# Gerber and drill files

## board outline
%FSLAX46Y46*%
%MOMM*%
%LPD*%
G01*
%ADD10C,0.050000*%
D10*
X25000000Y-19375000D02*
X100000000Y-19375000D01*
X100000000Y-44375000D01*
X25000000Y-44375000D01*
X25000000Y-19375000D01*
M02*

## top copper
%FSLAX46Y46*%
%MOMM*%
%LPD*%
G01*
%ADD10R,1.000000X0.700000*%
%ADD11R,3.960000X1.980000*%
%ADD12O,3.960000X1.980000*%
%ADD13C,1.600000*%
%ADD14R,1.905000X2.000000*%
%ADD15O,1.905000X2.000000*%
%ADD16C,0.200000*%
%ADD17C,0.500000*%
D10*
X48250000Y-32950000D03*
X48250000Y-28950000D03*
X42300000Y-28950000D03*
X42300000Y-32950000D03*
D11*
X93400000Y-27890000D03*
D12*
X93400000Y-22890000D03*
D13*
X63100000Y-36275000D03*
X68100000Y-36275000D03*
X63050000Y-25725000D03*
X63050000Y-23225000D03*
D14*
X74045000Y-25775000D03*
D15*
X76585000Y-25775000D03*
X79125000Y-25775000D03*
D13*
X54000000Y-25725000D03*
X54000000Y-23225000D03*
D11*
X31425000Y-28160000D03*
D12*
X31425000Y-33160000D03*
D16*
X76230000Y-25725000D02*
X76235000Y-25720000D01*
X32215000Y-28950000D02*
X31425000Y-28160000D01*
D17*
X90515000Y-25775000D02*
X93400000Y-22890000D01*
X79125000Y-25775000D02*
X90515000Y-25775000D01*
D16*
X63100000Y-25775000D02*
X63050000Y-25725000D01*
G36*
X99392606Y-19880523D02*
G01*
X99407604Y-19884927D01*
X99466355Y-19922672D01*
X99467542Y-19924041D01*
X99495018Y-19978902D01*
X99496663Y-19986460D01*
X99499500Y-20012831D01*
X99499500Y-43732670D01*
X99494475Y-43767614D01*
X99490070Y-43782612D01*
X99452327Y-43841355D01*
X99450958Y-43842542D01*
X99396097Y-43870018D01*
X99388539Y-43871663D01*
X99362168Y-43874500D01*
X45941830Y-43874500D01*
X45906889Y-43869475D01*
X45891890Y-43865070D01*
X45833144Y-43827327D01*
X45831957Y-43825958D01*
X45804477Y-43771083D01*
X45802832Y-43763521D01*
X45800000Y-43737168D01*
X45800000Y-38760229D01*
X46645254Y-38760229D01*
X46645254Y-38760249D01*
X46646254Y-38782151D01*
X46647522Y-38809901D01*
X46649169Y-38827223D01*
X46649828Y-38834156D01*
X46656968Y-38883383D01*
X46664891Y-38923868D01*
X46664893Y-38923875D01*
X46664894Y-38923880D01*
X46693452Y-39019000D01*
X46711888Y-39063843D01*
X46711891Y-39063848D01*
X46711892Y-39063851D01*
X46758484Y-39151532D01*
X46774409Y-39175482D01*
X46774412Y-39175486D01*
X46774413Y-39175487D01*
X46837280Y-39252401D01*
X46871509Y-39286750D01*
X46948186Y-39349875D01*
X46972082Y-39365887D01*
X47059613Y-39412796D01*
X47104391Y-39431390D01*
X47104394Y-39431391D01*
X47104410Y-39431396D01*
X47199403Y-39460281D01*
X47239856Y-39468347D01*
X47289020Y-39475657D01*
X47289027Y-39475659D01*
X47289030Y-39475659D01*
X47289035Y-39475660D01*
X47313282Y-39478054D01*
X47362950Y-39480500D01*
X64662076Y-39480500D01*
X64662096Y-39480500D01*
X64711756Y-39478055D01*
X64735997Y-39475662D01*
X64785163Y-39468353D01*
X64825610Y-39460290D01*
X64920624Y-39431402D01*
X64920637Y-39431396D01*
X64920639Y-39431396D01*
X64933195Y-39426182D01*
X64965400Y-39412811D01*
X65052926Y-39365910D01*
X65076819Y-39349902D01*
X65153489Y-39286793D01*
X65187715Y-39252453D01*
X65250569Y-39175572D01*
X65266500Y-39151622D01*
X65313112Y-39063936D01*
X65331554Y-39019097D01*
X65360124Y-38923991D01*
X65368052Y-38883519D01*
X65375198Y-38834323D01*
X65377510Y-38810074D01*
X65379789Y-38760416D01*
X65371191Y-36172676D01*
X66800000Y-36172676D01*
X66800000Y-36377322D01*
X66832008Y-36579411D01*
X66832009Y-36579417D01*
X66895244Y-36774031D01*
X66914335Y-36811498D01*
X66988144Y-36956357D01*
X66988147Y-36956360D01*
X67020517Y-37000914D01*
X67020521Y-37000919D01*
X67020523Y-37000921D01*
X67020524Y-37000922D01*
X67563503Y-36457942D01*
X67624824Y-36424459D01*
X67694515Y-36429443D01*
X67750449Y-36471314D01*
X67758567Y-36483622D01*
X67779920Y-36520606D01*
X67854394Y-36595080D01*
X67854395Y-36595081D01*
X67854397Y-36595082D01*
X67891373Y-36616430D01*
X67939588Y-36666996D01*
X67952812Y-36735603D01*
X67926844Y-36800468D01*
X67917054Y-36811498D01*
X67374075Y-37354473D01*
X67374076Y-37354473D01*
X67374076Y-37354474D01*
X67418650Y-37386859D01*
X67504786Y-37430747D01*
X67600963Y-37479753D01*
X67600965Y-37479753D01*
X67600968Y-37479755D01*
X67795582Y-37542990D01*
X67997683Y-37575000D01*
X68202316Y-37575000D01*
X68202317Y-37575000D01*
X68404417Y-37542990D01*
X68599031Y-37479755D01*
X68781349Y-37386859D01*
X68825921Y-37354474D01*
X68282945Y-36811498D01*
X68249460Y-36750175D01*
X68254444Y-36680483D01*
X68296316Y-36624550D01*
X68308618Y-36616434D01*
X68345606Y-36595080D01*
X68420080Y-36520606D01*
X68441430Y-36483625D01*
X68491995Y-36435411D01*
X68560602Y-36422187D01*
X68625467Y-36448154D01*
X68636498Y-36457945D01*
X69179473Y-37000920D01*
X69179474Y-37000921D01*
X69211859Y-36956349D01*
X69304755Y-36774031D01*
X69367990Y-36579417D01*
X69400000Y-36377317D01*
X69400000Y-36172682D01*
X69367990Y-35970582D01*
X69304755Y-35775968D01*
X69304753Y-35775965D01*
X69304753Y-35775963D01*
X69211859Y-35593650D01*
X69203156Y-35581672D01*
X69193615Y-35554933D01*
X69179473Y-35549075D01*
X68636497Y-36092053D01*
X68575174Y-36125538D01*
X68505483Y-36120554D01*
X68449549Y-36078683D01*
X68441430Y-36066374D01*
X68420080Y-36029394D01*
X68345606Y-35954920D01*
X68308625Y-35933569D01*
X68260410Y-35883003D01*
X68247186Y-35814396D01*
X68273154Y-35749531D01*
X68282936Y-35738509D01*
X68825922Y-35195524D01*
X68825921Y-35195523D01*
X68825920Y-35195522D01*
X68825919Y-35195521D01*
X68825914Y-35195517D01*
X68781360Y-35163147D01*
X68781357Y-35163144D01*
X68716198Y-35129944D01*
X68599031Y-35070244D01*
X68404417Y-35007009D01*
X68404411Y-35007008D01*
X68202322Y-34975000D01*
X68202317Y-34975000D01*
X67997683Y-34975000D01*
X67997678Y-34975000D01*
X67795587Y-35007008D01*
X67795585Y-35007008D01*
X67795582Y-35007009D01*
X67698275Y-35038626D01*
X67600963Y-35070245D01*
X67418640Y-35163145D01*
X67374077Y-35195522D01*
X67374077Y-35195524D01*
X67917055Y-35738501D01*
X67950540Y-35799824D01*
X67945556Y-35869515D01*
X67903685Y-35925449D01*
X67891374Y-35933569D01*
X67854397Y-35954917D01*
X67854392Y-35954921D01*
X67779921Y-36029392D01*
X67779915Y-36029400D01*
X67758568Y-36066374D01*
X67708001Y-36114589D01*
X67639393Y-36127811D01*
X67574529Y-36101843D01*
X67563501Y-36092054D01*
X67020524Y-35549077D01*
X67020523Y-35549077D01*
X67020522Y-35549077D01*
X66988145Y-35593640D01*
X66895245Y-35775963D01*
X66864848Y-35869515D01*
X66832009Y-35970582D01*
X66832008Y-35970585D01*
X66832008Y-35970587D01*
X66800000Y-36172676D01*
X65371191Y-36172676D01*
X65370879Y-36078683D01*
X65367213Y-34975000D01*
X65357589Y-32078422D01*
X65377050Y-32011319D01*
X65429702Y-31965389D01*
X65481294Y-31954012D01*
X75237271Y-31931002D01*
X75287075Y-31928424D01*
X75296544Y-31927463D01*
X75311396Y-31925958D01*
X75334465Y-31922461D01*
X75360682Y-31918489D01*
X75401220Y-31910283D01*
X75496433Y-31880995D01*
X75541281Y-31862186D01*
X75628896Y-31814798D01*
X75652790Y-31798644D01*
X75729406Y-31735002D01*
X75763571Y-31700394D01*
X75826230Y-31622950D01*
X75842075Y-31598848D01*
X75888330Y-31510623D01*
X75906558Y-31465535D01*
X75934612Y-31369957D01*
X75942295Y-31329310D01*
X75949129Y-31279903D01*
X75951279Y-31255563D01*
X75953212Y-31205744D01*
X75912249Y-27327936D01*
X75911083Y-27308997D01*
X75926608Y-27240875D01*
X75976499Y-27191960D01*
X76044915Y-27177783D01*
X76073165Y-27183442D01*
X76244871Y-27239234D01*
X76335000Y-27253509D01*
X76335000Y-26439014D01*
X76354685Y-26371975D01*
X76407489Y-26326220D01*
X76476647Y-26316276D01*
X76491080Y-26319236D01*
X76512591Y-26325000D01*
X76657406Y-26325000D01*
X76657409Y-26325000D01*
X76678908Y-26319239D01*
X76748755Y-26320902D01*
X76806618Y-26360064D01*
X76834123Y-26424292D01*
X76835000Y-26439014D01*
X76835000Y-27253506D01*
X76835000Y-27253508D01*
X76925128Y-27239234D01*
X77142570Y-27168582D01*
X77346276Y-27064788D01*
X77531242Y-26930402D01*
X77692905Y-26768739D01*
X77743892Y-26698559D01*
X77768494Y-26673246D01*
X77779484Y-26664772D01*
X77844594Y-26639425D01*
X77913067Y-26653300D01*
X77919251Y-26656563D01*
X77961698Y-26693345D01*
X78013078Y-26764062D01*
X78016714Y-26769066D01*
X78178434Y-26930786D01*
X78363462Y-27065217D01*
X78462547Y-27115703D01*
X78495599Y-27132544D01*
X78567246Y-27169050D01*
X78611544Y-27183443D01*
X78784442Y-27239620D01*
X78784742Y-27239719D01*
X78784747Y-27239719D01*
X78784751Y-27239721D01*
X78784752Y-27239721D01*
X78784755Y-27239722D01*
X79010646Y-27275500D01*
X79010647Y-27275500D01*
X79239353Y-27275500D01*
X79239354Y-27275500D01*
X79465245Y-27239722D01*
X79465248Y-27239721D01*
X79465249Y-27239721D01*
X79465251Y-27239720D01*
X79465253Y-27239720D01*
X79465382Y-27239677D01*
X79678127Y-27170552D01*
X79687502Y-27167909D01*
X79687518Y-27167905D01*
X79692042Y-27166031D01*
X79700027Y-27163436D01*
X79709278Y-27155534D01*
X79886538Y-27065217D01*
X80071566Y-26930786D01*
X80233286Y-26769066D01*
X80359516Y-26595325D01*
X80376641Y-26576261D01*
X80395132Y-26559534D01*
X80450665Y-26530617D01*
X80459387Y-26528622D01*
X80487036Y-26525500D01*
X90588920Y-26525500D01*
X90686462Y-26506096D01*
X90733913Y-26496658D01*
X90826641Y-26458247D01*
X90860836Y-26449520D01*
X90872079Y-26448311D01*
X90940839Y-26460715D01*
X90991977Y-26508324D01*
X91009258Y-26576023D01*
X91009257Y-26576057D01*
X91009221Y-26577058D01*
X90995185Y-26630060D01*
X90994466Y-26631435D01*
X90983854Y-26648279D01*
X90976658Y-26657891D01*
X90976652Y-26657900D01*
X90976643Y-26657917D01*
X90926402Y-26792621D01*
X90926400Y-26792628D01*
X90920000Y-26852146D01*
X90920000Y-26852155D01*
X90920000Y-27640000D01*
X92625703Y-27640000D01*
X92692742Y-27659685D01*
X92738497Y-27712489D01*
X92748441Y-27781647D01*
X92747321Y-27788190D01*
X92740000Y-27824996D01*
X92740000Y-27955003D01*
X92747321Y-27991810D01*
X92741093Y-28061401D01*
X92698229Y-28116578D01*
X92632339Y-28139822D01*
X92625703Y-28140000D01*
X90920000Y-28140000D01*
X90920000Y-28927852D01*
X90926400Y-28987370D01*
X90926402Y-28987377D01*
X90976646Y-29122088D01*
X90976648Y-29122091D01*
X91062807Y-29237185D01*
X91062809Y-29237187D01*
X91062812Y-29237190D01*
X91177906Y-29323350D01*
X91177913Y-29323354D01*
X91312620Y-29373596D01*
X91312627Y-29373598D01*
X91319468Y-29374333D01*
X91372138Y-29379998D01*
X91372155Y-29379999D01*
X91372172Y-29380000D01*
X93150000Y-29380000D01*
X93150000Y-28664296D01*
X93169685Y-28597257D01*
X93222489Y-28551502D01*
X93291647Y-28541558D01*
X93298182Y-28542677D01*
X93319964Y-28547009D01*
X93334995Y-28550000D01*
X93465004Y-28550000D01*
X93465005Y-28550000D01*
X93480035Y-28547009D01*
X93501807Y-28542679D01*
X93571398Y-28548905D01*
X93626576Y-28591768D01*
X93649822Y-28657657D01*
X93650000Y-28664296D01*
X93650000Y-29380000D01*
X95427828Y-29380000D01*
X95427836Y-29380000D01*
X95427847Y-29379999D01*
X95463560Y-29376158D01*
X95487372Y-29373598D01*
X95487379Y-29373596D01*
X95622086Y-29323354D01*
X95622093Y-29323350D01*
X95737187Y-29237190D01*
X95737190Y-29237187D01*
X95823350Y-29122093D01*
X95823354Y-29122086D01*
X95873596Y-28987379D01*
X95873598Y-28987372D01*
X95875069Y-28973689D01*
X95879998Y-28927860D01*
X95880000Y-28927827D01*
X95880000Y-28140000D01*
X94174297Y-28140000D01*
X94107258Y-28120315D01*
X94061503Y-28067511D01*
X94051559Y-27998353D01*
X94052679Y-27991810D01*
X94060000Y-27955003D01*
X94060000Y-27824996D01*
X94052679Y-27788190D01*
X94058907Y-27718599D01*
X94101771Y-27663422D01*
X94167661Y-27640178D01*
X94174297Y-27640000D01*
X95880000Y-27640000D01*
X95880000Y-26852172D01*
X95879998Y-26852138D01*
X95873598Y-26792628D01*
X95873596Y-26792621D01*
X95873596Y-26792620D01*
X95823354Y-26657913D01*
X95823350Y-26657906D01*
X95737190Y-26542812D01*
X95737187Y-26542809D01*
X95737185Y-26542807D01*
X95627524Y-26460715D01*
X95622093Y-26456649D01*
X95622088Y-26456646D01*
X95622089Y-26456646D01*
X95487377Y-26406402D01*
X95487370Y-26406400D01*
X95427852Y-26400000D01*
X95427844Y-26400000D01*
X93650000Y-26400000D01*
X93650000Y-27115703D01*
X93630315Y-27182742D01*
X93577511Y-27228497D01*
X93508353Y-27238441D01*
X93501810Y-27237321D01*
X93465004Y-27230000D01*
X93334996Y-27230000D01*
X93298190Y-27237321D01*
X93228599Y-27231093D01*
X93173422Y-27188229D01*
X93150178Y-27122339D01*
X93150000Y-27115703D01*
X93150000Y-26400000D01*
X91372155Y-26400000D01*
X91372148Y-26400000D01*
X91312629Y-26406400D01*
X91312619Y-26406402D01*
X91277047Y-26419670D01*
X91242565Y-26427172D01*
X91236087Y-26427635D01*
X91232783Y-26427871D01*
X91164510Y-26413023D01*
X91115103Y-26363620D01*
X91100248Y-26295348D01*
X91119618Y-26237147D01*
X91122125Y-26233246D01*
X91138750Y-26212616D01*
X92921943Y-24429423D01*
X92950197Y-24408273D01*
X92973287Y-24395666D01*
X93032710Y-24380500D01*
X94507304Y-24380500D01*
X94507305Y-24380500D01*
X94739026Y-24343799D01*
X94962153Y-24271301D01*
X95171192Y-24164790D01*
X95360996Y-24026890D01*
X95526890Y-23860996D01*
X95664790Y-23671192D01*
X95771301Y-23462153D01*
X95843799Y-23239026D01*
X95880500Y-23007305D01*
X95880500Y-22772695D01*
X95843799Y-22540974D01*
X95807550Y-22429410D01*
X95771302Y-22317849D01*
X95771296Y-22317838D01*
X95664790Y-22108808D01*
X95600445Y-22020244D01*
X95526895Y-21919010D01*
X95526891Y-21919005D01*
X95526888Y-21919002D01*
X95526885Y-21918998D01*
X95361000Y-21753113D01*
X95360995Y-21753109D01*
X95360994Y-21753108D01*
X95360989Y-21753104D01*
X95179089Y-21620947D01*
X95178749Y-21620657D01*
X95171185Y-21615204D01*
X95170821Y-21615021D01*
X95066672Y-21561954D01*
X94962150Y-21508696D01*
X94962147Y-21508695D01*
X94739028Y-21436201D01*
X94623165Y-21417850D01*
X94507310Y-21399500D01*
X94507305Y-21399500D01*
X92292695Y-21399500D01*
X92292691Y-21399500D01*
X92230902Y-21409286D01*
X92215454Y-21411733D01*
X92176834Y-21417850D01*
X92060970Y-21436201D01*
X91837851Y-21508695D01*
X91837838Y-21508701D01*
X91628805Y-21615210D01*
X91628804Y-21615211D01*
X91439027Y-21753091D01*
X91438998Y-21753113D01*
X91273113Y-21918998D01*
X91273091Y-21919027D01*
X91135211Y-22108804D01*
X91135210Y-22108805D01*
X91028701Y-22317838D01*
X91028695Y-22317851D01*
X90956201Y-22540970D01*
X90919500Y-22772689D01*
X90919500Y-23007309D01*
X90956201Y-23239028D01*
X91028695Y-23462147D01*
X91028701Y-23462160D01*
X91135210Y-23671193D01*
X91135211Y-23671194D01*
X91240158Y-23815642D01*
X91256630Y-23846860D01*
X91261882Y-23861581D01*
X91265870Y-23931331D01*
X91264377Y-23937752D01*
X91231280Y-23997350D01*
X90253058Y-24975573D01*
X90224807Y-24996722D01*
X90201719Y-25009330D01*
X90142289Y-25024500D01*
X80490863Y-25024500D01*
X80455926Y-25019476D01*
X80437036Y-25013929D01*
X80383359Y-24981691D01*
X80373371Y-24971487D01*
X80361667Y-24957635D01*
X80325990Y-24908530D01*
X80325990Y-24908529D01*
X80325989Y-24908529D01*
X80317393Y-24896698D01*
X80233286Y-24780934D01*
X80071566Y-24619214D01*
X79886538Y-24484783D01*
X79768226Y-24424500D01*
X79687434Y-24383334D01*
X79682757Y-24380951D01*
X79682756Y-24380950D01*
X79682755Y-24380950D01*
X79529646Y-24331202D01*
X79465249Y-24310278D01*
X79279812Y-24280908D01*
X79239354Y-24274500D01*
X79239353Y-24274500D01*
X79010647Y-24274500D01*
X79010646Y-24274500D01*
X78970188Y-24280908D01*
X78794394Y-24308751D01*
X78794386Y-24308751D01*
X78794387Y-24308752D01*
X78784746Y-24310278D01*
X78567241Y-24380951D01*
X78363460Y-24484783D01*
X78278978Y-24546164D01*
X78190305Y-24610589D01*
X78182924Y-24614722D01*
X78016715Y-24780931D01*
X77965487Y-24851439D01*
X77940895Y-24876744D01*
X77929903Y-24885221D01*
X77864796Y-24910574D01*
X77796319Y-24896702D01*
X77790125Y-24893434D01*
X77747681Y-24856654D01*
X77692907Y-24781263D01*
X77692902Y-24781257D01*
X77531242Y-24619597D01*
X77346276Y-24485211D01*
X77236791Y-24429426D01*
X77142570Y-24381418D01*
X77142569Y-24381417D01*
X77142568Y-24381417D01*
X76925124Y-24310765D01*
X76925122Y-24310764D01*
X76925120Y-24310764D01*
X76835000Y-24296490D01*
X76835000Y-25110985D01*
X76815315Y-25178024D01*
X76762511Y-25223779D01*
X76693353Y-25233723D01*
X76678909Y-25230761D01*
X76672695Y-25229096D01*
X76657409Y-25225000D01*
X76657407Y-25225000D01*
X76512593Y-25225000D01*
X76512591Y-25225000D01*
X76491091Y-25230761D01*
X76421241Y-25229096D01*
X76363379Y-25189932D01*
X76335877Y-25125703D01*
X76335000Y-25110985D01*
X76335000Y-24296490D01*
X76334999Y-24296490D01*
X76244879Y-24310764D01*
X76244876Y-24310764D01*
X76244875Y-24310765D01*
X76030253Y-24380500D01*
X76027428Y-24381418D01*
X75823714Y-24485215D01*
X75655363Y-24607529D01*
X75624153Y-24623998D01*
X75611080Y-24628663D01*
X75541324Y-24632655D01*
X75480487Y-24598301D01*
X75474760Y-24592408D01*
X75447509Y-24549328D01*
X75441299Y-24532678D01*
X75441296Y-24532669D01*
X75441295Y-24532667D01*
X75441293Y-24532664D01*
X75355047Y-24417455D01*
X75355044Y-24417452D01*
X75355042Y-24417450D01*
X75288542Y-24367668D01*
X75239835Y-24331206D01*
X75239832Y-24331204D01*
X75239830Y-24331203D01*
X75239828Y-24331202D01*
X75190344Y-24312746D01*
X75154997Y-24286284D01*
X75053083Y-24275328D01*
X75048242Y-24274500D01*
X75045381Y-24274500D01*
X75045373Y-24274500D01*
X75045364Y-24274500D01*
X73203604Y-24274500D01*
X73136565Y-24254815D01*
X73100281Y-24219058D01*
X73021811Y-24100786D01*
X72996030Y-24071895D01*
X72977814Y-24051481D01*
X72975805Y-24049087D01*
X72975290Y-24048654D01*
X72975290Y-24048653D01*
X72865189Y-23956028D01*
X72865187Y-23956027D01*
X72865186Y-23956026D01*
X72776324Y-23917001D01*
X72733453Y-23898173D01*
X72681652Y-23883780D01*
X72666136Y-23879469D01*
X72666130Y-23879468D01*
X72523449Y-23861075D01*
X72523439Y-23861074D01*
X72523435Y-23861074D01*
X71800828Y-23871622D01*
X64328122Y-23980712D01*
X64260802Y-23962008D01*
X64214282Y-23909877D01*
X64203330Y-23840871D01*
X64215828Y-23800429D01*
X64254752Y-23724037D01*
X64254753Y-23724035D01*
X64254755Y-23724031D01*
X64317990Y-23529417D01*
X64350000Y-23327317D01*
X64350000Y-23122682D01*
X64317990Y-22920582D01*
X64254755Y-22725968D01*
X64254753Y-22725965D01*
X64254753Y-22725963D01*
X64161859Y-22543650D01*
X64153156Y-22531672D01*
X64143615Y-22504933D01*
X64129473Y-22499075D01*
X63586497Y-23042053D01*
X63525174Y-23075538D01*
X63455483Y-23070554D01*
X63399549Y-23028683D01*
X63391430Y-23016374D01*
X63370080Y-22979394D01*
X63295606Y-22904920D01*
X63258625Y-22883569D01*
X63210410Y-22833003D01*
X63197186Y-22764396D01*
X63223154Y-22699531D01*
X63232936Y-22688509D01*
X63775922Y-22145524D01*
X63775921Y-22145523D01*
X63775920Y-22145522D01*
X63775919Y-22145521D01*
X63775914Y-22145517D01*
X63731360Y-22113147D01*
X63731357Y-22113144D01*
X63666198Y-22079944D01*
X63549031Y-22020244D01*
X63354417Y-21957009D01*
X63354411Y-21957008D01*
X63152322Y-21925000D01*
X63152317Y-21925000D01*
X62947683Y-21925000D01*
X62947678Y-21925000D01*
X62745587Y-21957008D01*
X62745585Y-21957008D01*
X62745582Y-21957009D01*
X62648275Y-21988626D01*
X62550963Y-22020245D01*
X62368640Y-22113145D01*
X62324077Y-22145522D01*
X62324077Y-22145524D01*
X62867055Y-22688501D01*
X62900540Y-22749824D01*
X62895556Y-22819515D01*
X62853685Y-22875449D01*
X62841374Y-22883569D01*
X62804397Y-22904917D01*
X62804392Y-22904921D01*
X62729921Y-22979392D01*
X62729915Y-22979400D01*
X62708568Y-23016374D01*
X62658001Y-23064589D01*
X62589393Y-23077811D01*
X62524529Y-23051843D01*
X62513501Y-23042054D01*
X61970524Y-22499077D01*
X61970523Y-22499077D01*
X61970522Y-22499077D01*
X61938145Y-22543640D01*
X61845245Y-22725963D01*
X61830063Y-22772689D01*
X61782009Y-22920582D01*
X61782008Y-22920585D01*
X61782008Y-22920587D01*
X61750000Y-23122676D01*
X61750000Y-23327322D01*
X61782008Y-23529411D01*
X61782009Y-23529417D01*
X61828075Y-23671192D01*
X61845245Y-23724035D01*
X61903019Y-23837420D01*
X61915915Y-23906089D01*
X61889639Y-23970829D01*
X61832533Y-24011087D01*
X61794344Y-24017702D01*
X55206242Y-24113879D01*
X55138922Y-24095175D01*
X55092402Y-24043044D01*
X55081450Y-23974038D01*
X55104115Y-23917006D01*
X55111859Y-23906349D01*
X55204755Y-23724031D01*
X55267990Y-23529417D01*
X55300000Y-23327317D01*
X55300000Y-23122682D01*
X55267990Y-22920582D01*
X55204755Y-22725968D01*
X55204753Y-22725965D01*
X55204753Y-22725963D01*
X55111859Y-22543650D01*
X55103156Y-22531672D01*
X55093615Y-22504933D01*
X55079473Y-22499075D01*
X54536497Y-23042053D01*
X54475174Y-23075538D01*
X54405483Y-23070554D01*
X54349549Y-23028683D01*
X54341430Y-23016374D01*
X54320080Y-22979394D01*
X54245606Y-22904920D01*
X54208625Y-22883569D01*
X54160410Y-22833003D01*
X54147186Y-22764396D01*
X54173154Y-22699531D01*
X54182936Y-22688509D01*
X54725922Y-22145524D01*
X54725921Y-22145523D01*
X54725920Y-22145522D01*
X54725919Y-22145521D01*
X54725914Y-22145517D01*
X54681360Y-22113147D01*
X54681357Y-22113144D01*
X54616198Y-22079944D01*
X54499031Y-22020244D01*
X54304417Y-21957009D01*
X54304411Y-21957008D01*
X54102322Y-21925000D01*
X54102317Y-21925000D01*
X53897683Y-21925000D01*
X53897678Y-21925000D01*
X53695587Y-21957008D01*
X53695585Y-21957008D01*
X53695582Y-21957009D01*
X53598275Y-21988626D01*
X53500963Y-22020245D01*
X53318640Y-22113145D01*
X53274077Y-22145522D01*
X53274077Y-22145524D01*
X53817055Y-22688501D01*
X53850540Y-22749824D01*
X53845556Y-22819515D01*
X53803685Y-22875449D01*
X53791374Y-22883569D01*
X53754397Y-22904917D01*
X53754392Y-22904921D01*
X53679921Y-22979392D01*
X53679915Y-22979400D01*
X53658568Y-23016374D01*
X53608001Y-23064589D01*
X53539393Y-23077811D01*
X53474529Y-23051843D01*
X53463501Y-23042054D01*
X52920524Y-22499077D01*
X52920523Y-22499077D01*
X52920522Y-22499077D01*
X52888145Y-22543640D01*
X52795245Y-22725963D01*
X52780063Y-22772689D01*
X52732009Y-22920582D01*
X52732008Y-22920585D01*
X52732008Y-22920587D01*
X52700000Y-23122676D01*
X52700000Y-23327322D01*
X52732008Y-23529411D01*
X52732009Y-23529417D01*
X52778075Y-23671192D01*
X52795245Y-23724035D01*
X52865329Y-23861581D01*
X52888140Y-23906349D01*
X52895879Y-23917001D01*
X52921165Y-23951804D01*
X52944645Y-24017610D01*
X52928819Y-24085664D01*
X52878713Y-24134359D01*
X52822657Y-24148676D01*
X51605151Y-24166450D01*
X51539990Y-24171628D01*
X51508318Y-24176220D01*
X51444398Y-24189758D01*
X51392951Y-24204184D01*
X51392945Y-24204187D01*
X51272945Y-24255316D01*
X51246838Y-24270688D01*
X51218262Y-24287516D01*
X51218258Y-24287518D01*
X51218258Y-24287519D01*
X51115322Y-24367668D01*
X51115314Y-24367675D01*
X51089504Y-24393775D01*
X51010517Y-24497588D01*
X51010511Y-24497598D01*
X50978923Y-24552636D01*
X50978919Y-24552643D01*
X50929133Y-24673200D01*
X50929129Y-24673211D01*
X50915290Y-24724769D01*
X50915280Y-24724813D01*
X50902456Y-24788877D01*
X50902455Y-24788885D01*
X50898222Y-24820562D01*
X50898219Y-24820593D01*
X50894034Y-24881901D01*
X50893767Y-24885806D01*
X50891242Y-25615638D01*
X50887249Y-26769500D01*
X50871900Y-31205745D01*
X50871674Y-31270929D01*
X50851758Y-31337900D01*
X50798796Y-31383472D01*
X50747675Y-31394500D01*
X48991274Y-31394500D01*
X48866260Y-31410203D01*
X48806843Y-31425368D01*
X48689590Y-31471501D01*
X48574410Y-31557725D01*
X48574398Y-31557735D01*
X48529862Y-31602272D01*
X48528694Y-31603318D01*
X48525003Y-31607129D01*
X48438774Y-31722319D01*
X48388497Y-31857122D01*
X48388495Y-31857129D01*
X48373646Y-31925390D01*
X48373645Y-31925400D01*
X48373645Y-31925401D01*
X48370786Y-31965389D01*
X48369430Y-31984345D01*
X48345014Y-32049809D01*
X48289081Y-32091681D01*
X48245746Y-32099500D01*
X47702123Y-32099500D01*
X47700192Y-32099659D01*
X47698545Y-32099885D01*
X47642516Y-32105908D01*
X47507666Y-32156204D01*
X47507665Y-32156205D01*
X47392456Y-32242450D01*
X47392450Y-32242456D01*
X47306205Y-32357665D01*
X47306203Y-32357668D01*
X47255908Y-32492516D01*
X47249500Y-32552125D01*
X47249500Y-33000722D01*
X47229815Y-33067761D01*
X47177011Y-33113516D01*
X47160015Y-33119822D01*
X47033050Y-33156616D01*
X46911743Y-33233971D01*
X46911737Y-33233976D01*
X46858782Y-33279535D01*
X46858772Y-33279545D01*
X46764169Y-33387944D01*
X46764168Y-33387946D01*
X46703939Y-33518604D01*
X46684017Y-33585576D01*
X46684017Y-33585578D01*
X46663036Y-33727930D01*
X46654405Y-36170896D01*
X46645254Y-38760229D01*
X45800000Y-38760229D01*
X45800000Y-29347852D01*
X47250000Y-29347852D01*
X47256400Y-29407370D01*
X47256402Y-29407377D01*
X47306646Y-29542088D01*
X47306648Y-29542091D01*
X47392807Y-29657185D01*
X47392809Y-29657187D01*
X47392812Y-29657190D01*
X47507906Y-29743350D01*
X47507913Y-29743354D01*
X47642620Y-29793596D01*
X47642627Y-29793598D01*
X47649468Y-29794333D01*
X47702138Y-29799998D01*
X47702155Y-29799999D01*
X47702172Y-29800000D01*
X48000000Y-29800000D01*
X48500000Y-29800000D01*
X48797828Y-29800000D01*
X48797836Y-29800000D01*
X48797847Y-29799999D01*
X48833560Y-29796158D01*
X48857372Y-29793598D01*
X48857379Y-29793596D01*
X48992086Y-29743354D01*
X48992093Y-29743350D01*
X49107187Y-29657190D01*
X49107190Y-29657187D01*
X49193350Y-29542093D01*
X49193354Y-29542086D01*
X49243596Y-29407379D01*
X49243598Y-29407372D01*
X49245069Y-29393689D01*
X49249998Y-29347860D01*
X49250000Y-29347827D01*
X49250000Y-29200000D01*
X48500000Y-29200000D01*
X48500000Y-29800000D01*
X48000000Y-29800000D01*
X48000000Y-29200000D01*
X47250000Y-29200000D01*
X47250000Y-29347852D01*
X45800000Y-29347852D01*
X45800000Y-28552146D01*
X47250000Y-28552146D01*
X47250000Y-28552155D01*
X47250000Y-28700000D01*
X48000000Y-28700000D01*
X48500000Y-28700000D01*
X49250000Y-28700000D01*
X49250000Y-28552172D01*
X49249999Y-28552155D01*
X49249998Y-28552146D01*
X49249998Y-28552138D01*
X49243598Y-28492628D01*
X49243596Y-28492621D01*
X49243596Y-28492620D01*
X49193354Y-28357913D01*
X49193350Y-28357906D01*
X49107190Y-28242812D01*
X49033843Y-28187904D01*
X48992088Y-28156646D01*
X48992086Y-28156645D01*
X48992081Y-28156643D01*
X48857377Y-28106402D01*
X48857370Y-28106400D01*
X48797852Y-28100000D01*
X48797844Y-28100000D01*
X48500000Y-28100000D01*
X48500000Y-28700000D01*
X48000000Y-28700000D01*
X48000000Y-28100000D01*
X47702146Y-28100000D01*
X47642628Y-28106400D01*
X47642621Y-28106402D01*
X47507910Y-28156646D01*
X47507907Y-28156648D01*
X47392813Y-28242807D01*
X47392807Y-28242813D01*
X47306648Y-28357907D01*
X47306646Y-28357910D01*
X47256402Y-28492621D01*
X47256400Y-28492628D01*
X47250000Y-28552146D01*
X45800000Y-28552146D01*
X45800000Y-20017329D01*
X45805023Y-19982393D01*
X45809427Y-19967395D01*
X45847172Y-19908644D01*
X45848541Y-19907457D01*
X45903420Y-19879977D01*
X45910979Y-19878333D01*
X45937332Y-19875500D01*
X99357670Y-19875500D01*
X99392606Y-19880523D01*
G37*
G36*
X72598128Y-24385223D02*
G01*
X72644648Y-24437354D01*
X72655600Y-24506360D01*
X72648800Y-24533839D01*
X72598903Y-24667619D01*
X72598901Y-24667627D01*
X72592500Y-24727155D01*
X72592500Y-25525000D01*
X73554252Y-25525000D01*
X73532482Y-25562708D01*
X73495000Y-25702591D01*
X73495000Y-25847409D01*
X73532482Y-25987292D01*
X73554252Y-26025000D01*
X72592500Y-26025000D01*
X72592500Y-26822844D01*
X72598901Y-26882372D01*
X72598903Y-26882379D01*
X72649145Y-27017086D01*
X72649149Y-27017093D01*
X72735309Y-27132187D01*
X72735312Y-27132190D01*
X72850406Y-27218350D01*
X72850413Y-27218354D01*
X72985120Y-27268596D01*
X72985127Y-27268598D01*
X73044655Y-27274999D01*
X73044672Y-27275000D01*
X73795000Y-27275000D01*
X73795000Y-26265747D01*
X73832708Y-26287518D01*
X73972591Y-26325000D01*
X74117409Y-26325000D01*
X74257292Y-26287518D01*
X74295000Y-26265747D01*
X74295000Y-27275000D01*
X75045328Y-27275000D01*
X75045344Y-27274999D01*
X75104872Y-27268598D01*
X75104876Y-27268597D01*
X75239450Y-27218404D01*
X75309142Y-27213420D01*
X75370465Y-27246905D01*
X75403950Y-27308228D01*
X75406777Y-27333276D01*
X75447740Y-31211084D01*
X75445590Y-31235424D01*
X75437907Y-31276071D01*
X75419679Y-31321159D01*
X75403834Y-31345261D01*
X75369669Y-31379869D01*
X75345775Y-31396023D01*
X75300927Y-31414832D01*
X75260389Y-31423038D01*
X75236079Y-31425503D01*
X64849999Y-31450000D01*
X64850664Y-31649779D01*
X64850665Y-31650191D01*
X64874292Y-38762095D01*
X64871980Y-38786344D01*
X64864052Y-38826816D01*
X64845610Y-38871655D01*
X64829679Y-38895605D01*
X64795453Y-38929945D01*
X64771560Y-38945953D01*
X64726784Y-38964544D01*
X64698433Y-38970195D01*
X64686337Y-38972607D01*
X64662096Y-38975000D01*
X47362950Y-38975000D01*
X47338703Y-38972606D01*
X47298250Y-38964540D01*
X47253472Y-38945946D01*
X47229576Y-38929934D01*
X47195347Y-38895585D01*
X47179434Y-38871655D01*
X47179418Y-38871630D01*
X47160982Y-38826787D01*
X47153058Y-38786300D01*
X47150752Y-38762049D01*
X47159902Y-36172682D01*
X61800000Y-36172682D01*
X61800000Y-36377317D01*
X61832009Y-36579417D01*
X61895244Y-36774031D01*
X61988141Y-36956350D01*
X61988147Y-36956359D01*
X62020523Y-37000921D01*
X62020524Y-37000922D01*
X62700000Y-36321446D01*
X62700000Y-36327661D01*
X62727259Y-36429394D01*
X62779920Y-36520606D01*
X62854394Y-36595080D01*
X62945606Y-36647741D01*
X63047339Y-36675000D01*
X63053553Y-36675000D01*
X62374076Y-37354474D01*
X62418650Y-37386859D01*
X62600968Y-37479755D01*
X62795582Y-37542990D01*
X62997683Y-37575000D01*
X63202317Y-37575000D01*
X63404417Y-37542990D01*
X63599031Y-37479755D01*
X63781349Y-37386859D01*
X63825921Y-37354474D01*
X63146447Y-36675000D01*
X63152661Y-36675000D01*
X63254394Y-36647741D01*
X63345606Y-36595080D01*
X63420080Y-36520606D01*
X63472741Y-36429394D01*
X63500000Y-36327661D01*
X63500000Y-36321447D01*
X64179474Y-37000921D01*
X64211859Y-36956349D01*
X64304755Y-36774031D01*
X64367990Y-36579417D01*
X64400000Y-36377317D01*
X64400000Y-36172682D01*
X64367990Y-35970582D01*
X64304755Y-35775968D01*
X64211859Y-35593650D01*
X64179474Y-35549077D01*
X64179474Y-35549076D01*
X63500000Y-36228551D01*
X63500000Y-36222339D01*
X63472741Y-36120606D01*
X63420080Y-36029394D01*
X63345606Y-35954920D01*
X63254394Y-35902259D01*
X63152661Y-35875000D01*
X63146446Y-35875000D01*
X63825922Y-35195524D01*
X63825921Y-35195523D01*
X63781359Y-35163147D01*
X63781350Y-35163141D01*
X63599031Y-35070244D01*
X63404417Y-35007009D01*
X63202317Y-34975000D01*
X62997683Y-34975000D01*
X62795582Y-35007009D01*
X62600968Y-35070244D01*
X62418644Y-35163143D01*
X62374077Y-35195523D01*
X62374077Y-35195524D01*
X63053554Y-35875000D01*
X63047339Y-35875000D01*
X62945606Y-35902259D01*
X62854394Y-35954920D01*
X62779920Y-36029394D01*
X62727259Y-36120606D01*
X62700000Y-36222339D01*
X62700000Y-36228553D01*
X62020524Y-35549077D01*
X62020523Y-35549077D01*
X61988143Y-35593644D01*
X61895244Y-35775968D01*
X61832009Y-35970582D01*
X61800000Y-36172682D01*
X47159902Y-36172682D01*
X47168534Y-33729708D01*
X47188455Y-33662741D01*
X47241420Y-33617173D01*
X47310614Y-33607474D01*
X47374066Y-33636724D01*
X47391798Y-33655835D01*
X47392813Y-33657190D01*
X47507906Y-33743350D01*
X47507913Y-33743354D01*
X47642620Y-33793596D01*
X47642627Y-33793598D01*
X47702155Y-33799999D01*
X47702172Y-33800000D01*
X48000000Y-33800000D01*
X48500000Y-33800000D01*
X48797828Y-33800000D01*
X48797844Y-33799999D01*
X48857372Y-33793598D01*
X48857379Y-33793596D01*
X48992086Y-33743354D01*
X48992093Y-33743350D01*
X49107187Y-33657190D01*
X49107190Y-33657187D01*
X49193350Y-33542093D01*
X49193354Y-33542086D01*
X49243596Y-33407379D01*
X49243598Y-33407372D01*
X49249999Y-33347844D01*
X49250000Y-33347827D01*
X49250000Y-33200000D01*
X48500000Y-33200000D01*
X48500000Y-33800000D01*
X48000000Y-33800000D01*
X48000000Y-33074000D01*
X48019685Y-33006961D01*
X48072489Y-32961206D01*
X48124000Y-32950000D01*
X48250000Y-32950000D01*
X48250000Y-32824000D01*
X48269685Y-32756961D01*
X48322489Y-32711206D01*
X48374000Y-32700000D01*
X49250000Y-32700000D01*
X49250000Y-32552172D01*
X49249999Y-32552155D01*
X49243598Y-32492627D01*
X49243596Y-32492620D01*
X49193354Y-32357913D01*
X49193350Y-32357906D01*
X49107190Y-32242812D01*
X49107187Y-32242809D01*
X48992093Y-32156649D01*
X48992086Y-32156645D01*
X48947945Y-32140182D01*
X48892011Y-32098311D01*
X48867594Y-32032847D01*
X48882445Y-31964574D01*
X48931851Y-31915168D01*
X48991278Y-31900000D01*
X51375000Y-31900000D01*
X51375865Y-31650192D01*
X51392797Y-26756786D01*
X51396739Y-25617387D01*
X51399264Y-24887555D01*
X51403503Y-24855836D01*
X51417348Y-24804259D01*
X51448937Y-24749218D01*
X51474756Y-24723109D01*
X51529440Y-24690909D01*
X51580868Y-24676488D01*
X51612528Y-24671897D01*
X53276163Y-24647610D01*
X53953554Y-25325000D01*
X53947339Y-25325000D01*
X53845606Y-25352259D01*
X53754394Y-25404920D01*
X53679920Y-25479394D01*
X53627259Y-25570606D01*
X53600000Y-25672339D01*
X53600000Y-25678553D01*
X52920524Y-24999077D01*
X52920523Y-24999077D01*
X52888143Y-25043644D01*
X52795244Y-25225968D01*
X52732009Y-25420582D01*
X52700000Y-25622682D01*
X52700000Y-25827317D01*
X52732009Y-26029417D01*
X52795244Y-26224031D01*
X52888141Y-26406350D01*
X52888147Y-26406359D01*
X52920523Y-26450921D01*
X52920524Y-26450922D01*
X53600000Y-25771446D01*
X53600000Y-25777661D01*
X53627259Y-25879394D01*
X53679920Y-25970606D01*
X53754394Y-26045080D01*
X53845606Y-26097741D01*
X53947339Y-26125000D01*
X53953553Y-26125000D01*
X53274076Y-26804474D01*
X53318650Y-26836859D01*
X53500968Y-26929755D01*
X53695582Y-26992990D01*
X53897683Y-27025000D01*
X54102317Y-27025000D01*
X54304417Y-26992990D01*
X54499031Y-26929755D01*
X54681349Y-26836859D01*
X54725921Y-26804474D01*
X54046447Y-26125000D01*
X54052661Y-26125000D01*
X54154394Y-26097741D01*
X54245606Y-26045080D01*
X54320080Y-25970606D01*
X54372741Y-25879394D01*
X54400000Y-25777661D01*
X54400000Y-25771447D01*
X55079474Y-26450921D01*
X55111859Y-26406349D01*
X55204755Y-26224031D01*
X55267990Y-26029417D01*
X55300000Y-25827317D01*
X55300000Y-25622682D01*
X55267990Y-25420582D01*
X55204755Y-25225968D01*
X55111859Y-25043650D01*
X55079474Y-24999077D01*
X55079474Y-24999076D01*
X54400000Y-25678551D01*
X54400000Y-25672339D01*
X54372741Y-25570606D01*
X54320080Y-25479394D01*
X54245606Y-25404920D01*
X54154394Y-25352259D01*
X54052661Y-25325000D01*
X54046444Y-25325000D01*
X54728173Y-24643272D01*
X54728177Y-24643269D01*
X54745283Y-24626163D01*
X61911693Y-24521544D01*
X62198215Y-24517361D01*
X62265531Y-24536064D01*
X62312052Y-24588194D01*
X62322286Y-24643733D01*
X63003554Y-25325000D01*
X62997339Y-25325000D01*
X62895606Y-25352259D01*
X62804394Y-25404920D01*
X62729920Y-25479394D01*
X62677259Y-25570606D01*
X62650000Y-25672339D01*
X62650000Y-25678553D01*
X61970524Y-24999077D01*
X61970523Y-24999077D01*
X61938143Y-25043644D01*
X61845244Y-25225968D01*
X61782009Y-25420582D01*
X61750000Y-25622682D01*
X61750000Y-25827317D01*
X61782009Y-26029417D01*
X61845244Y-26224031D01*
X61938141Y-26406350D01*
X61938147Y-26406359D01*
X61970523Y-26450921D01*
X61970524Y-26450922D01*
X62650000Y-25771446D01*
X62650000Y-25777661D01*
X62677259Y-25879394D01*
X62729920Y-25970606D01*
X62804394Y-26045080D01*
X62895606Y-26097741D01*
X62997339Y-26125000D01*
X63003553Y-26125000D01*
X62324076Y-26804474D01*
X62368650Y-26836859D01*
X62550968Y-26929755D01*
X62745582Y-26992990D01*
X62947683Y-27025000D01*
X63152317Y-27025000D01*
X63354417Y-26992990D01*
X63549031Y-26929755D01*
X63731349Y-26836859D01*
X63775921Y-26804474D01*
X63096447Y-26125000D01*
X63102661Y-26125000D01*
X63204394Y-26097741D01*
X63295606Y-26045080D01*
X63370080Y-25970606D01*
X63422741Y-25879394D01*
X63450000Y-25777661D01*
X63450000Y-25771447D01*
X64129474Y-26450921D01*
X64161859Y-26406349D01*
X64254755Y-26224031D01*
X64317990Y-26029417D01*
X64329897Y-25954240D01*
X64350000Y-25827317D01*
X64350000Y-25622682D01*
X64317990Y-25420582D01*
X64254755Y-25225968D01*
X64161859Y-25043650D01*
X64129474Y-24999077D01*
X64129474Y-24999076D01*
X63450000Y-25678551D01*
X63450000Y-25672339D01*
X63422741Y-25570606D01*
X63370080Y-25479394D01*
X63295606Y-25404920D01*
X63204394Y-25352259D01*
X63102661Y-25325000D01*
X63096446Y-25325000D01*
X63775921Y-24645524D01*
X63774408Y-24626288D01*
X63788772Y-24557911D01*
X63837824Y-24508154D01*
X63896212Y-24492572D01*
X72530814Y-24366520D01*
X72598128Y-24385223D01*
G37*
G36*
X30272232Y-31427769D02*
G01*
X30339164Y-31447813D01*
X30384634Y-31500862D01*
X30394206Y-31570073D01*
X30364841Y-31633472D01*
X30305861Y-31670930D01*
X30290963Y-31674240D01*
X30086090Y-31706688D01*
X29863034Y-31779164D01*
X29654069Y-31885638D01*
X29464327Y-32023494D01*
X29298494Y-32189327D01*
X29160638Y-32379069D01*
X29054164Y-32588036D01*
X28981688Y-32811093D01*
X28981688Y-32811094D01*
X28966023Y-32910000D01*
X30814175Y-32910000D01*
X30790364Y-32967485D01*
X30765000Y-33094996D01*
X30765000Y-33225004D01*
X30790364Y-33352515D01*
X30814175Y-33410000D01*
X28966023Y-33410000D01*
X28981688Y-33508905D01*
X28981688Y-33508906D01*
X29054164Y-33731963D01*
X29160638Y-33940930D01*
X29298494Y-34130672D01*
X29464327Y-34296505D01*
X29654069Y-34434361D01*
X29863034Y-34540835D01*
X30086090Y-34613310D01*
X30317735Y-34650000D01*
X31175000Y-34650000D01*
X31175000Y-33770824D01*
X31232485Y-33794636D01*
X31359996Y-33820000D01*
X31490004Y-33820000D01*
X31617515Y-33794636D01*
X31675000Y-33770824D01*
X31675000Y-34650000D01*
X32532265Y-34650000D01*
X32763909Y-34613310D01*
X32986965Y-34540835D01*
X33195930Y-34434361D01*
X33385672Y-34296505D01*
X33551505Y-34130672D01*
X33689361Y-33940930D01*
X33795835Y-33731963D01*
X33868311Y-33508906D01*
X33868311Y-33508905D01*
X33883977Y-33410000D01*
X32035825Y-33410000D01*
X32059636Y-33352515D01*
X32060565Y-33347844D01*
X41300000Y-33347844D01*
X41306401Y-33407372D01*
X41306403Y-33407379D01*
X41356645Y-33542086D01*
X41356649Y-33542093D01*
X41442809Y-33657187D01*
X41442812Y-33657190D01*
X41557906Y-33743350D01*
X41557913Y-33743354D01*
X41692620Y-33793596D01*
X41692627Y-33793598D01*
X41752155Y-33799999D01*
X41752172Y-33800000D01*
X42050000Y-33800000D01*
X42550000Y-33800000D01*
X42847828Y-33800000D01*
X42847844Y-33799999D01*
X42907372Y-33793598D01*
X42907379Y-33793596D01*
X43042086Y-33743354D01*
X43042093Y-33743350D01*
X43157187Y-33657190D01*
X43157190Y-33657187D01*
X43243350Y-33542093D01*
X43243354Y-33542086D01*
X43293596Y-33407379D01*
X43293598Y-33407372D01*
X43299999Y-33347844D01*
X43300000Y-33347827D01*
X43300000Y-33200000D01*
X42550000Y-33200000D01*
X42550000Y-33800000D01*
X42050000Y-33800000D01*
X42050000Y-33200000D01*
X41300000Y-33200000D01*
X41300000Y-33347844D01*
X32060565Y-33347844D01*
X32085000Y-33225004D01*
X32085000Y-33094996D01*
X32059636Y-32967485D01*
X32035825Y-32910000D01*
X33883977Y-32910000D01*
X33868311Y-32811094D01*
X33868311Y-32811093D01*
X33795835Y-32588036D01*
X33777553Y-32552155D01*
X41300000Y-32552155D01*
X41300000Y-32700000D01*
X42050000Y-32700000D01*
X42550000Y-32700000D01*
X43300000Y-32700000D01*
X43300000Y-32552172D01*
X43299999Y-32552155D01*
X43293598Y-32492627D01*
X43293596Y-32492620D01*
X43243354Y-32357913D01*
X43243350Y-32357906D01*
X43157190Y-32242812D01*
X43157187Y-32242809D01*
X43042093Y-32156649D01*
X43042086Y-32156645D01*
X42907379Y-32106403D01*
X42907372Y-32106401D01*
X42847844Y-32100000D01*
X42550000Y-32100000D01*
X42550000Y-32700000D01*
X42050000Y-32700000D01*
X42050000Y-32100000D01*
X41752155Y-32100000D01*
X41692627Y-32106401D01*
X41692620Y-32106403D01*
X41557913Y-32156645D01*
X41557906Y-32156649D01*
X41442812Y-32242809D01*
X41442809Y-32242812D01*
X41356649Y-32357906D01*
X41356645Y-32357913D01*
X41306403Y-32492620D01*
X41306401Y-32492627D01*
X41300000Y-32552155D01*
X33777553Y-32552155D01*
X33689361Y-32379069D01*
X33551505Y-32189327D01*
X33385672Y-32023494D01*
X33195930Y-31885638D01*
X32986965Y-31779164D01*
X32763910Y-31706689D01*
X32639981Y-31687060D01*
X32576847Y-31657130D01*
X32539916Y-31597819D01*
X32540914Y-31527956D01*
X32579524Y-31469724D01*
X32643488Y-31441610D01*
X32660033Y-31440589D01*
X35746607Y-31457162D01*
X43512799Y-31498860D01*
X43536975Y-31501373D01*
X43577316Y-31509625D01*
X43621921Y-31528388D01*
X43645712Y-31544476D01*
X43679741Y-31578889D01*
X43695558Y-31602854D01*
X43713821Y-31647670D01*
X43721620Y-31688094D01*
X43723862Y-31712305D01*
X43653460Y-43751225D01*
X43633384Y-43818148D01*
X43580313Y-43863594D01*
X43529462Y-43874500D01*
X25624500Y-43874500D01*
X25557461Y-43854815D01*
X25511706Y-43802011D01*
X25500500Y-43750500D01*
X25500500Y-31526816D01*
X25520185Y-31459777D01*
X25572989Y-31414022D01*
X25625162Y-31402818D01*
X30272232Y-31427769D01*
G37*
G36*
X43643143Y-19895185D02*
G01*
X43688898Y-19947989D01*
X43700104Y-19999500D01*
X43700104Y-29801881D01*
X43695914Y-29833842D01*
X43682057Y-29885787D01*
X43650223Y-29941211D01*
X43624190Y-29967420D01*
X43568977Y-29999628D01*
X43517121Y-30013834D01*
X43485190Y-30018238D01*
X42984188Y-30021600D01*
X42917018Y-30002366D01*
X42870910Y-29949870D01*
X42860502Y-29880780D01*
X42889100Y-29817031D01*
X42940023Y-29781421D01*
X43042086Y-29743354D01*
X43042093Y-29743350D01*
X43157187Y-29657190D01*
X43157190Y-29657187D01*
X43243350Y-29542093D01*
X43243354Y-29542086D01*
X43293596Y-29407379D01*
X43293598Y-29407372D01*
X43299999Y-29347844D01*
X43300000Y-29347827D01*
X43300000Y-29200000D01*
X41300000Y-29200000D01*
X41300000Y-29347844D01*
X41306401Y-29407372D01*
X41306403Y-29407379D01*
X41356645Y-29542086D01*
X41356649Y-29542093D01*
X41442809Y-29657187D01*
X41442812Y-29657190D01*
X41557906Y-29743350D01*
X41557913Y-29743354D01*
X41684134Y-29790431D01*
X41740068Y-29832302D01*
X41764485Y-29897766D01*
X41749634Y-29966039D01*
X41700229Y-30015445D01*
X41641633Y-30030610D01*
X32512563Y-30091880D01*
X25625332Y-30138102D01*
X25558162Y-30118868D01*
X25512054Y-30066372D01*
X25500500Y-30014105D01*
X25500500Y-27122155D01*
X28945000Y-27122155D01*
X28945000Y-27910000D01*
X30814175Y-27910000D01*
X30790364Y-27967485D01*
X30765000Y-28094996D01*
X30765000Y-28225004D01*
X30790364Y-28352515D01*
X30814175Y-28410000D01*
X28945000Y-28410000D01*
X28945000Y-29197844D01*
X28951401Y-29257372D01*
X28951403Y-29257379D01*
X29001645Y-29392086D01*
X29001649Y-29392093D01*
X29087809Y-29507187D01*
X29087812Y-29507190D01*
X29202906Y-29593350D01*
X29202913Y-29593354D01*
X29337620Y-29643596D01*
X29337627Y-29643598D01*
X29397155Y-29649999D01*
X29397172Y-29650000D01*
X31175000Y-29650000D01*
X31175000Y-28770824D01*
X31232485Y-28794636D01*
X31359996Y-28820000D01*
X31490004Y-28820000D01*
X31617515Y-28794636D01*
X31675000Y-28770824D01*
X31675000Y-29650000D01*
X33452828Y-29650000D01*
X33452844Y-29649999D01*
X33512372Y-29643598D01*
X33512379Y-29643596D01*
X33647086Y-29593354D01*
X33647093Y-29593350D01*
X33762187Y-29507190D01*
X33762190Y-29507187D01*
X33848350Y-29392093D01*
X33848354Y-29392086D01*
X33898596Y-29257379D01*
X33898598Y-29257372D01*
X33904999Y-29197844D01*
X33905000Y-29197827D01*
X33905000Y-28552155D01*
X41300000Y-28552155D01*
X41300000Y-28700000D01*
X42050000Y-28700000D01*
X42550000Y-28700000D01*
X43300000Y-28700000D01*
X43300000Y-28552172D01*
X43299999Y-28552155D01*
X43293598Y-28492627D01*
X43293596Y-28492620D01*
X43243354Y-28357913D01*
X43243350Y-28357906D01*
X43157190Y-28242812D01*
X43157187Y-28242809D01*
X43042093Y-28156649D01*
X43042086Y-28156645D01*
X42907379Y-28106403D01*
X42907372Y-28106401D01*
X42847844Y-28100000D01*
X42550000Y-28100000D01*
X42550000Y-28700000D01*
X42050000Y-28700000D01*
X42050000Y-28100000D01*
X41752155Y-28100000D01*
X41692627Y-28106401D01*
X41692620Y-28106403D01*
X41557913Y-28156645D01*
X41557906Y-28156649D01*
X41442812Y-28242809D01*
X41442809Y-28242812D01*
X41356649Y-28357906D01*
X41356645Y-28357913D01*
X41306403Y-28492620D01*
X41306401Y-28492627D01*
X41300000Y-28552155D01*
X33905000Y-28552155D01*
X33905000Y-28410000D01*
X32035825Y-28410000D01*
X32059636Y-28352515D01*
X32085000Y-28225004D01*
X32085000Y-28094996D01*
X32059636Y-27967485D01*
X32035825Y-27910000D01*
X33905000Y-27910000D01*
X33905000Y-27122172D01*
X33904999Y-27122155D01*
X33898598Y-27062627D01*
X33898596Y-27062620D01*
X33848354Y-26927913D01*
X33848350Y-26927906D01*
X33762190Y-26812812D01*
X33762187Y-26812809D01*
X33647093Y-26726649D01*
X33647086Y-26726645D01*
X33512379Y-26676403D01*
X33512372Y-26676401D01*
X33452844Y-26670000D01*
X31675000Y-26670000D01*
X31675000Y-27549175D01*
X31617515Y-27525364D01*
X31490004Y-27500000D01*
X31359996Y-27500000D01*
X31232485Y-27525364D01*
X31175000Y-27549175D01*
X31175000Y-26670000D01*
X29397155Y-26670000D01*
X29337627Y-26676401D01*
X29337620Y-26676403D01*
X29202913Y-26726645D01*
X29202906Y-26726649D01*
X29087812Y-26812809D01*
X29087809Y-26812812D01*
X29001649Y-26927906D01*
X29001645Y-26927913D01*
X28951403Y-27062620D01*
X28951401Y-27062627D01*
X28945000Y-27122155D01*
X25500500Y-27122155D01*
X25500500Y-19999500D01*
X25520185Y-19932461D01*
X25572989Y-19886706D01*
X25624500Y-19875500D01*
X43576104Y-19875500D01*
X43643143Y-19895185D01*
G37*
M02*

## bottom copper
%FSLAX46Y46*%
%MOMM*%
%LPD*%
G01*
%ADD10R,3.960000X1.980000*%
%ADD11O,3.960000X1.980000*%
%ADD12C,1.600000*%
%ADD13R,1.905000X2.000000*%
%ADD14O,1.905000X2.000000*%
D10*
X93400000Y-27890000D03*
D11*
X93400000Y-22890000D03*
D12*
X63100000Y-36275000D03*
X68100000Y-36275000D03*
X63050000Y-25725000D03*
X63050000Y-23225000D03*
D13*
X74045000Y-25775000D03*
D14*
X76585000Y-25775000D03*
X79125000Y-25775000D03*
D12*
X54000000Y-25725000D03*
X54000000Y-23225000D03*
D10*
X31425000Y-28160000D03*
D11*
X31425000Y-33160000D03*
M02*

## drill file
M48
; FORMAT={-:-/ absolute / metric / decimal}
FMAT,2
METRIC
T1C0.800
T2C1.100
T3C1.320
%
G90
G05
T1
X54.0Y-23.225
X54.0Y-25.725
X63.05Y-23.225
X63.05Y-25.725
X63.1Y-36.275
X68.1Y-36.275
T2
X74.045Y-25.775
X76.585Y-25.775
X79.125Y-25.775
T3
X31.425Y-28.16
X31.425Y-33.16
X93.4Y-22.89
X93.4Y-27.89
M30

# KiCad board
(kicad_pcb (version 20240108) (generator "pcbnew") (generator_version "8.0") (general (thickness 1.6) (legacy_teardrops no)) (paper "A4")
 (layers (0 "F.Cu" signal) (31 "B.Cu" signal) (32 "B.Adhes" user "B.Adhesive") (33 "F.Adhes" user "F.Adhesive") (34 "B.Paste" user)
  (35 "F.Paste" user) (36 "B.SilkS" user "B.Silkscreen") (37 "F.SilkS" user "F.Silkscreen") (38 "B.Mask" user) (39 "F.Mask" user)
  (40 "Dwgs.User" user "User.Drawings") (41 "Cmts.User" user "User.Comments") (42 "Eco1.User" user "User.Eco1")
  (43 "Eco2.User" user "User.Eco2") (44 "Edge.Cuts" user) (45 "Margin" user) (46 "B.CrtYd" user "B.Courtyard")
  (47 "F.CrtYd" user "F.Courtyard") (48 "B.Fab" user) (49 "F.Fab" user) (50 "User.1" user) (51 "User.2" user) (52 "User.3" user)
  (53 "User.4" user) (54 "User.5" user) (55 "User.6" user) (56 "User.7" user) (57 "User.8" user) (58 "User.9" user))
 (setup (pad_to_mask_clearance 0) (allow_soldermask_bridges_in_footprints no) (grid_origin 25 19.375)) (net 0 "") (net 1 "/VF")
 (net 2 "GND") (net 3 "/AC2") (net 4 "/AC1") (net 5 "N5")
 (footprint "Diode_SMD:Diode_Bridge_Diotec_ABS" (layer "F.Cu") (at 45.275 30.95 180)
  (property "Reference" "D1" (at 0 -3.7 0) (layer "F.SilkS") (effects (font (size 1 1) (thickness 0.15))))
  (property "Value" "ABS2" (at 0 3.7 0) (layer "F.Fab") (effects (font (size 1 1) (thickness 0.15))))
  (pad "1" smd rect (at -2.975 -2 180) (size 1 0.7) (layers "F.Cu" "F.Paste" "F.Mask") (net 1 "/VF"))
  (pad "2" smd rect (at -2.975 2 180) (size 1 0.7) (layers "F.Cu" "F.Paste" "F.Mask") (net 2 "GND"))
  (pad "3" smd rect (at 2.975 2 180) (size 1 0.7) (layers "F.Cu" "F.Paste" "F.Mask") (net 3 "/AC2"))
  (pad "4" smd rect (at 2.975 -2 180) (size 1 0.7) (layers "F.Cu" "F.Paste" "F.Mask") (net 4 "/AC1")))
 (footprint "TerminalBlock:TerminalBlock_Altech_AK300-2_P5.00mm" (layer "F.Cu") (at 93.4 27.89 90)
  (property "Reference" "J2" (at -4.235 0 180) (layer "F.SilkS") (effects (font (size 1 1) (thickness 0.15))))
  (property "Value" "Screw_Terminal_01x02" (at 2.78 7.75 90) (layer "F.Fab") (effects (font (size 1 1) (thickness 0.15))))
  (pad "1" thru_hole rect (at 0 0 90) (size 1.98 3.96) (drill 1.32) (layers "*.Cu" "*.Mask") (remove_unused_layers no) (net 2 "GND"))
  (pad "2" thru_hole oval (at 5 0 90) (size 1.98 3.96) (drill 1.32) (layers "*.Cu" "*.Mask") (remove_unused_layers no) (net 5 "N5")))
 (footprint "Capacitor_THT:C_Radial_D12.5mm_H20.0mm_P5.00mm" (layer "F.Cu") (at 63.1 36.275)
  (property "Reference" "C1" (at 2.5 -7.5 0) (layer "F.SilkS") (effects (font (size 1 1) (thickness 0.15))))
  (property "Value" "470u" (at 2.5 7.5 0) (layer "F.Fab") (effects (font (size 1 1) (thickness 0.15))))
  (pad "1" thru_hole circle (at 0 0) (size 1.6 1.6) (drill 0.8) (layers "*.Cu" "*.Mask") (remove_unused_layers no) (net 1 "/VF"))
  (pad "2" thru_hole circle (at 5 0) (size 1.6 1.6) (drill 0.8) (layers "*.Cu" "*.Mask") (remove_unused_layers no) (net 2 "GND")))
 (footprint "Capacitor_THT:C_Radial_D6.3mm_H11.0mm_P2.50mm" (layer "F.Cu") (at 63.05 25.725 90)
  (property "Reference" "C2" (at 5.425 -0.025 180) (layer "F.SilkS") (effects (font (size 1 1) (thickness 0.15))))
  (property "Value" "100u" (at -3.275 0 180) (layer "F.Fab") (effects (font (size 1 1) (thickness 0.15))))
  (pad "1" thru_hole circle (at 0 0 90) (size 1.6 1.6) (drill 0.8) (layers "*.Cu" "*.Mask") (remove_unused_layers no) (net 1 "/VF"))
  (pad "2" thru_hole circle (at 2.5 0 90) (size 1.6 1.6) (drill 0.8) (layers "*.Cu" "*.Mask") (remove_unused_layers no) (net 2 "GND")))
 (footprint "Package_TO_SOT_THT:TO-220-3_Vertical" (layer "F.Cu") (at 74.045 25.775)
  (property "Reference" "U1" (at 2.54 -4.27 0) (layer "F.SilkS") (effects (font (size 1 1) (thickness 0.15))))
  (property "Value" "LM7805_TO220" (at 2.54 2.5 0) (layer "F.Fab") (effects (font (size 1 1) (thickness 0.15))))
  (pad "1" thru_hole rect (at 0 0) (size 1.905 2) (drill 1.1) (layers "*.Cu" "*.Mask") (remove_unused_layers no) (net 1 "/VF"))
  (pad "2" thru_hole oval (at 2.54 0) (size 1.905 2) (drill 1.1) (layers "*.Cu" "*.Mask") (remove_unused_layers no) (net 2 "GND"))
  (pad "3" thru_hole oval (at 5.08 0) (size 1.905 2) (drill 1.1) (layers "*.Cu" "*.Mask") (remove_unused_layers no) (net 5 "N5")))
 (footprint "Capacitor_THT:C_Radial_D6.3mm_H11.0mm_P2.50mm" (layer "F.Cu") (at 54 25.725 90)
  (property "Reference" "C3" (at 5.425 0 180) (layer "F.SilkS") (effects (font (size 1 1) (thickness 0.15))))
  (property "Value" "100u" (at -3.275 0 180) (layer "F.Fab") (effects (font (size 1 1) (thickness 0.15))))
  (pad "1" thru_hole circle (at 0 0 90) (size 1.6 1.6) (drill 0.8) (layers "*.Cu" "*.Mask") (remove_unused_layers no) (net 1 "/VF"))
  (pad "2" thru_hole circle (at 2.5 0 90) (size 1.6 1.6) (drill 0.8) (layers "*.Cu" "*.Mask") (remove_unused_layers no) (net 2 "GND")))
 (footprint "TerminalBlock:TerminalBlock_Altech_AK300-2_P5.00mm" (layer "F.Cu") (at 31.425 28.16 -90)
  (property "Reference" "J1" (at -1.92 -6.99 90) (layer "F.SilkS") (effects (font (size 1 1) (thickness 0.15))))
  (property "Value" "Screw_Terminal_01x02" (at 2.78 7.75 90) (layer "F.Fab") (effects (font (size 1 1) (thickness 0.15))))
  (pad "1" thru_hole rect (at 0 0 270) (size 1.98 3.96) (drill 1.32) (layers "*.Cu" "*.Mask") (remove_unused_layers no) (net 3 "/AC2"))
  (pad "2" thru_hole oval (at 5 0 270) (size 1.98 3.96) (drill 1.32) (layers "*.Cu" "*.Mask") (remove_unused_layers no) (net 4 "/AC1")))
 (gr_rect (start 25 19.375) (end 100 44.375) (stroke (width 0.05) (type default)) (fill none) (layer "Edge.Cuts"))
 (segment (start 76.23 25.725) (end 76.235 25.72) (width 0.2) (layer "F.Cu") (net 2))
 (segment (start 32.215 28.95) (end 31.425 28.16) (width 0.2) (layer "F.Cu") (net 3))
 (segment (start 90.515 25.775) (end 93.4 22.89) (width 0.5) (layer "F.Cu") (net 5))
 (segment (start 79.125 25.775) (end 90.515 25.775) (width 0.5) (layer "F.Cu") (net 5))
 (segment (start 63.1 25.775) (end 63.05 25.725) (width 0.2) (layer "F.Cu") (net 1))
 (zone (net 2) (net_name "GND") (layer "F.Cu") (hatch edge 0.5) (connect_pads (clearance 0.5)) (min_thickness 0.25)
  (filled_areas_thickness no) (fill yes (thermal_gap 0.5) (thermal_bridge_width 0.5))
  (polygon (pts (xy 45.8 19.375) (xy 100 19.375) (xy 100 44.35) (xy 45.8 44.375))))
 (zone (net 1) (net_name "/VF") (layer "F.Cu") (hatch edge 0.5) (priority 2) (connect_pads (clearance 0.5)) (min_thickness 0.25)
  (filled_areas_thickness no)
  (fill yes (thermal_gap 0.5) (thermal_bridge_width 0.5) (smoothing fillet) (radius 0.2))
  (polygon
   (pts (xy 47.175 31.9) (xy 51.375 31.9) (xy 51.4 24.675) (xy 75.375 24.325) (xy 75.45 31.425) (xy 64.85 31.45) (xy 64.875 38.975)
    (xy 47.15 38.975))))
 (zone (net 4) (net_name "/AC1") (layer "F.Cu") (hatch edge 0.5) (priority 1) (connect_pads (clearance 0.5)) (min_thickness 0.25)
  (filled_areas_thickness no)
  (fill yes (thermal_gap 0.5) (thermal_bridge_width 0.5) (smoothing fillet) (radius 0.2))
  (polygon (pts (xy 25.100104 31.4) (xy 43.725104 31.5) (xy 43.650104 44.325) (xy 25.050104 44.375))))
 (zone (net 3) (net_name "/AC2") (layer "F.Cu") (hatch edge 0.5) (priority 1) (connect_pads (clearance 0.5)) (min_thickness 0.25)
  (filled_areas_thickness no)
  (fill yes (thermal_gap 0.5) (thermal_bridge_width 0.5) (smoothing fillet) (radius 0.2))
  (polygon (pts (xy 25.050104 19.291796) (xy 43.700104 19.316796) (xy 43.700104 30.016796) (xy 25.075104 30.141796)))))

